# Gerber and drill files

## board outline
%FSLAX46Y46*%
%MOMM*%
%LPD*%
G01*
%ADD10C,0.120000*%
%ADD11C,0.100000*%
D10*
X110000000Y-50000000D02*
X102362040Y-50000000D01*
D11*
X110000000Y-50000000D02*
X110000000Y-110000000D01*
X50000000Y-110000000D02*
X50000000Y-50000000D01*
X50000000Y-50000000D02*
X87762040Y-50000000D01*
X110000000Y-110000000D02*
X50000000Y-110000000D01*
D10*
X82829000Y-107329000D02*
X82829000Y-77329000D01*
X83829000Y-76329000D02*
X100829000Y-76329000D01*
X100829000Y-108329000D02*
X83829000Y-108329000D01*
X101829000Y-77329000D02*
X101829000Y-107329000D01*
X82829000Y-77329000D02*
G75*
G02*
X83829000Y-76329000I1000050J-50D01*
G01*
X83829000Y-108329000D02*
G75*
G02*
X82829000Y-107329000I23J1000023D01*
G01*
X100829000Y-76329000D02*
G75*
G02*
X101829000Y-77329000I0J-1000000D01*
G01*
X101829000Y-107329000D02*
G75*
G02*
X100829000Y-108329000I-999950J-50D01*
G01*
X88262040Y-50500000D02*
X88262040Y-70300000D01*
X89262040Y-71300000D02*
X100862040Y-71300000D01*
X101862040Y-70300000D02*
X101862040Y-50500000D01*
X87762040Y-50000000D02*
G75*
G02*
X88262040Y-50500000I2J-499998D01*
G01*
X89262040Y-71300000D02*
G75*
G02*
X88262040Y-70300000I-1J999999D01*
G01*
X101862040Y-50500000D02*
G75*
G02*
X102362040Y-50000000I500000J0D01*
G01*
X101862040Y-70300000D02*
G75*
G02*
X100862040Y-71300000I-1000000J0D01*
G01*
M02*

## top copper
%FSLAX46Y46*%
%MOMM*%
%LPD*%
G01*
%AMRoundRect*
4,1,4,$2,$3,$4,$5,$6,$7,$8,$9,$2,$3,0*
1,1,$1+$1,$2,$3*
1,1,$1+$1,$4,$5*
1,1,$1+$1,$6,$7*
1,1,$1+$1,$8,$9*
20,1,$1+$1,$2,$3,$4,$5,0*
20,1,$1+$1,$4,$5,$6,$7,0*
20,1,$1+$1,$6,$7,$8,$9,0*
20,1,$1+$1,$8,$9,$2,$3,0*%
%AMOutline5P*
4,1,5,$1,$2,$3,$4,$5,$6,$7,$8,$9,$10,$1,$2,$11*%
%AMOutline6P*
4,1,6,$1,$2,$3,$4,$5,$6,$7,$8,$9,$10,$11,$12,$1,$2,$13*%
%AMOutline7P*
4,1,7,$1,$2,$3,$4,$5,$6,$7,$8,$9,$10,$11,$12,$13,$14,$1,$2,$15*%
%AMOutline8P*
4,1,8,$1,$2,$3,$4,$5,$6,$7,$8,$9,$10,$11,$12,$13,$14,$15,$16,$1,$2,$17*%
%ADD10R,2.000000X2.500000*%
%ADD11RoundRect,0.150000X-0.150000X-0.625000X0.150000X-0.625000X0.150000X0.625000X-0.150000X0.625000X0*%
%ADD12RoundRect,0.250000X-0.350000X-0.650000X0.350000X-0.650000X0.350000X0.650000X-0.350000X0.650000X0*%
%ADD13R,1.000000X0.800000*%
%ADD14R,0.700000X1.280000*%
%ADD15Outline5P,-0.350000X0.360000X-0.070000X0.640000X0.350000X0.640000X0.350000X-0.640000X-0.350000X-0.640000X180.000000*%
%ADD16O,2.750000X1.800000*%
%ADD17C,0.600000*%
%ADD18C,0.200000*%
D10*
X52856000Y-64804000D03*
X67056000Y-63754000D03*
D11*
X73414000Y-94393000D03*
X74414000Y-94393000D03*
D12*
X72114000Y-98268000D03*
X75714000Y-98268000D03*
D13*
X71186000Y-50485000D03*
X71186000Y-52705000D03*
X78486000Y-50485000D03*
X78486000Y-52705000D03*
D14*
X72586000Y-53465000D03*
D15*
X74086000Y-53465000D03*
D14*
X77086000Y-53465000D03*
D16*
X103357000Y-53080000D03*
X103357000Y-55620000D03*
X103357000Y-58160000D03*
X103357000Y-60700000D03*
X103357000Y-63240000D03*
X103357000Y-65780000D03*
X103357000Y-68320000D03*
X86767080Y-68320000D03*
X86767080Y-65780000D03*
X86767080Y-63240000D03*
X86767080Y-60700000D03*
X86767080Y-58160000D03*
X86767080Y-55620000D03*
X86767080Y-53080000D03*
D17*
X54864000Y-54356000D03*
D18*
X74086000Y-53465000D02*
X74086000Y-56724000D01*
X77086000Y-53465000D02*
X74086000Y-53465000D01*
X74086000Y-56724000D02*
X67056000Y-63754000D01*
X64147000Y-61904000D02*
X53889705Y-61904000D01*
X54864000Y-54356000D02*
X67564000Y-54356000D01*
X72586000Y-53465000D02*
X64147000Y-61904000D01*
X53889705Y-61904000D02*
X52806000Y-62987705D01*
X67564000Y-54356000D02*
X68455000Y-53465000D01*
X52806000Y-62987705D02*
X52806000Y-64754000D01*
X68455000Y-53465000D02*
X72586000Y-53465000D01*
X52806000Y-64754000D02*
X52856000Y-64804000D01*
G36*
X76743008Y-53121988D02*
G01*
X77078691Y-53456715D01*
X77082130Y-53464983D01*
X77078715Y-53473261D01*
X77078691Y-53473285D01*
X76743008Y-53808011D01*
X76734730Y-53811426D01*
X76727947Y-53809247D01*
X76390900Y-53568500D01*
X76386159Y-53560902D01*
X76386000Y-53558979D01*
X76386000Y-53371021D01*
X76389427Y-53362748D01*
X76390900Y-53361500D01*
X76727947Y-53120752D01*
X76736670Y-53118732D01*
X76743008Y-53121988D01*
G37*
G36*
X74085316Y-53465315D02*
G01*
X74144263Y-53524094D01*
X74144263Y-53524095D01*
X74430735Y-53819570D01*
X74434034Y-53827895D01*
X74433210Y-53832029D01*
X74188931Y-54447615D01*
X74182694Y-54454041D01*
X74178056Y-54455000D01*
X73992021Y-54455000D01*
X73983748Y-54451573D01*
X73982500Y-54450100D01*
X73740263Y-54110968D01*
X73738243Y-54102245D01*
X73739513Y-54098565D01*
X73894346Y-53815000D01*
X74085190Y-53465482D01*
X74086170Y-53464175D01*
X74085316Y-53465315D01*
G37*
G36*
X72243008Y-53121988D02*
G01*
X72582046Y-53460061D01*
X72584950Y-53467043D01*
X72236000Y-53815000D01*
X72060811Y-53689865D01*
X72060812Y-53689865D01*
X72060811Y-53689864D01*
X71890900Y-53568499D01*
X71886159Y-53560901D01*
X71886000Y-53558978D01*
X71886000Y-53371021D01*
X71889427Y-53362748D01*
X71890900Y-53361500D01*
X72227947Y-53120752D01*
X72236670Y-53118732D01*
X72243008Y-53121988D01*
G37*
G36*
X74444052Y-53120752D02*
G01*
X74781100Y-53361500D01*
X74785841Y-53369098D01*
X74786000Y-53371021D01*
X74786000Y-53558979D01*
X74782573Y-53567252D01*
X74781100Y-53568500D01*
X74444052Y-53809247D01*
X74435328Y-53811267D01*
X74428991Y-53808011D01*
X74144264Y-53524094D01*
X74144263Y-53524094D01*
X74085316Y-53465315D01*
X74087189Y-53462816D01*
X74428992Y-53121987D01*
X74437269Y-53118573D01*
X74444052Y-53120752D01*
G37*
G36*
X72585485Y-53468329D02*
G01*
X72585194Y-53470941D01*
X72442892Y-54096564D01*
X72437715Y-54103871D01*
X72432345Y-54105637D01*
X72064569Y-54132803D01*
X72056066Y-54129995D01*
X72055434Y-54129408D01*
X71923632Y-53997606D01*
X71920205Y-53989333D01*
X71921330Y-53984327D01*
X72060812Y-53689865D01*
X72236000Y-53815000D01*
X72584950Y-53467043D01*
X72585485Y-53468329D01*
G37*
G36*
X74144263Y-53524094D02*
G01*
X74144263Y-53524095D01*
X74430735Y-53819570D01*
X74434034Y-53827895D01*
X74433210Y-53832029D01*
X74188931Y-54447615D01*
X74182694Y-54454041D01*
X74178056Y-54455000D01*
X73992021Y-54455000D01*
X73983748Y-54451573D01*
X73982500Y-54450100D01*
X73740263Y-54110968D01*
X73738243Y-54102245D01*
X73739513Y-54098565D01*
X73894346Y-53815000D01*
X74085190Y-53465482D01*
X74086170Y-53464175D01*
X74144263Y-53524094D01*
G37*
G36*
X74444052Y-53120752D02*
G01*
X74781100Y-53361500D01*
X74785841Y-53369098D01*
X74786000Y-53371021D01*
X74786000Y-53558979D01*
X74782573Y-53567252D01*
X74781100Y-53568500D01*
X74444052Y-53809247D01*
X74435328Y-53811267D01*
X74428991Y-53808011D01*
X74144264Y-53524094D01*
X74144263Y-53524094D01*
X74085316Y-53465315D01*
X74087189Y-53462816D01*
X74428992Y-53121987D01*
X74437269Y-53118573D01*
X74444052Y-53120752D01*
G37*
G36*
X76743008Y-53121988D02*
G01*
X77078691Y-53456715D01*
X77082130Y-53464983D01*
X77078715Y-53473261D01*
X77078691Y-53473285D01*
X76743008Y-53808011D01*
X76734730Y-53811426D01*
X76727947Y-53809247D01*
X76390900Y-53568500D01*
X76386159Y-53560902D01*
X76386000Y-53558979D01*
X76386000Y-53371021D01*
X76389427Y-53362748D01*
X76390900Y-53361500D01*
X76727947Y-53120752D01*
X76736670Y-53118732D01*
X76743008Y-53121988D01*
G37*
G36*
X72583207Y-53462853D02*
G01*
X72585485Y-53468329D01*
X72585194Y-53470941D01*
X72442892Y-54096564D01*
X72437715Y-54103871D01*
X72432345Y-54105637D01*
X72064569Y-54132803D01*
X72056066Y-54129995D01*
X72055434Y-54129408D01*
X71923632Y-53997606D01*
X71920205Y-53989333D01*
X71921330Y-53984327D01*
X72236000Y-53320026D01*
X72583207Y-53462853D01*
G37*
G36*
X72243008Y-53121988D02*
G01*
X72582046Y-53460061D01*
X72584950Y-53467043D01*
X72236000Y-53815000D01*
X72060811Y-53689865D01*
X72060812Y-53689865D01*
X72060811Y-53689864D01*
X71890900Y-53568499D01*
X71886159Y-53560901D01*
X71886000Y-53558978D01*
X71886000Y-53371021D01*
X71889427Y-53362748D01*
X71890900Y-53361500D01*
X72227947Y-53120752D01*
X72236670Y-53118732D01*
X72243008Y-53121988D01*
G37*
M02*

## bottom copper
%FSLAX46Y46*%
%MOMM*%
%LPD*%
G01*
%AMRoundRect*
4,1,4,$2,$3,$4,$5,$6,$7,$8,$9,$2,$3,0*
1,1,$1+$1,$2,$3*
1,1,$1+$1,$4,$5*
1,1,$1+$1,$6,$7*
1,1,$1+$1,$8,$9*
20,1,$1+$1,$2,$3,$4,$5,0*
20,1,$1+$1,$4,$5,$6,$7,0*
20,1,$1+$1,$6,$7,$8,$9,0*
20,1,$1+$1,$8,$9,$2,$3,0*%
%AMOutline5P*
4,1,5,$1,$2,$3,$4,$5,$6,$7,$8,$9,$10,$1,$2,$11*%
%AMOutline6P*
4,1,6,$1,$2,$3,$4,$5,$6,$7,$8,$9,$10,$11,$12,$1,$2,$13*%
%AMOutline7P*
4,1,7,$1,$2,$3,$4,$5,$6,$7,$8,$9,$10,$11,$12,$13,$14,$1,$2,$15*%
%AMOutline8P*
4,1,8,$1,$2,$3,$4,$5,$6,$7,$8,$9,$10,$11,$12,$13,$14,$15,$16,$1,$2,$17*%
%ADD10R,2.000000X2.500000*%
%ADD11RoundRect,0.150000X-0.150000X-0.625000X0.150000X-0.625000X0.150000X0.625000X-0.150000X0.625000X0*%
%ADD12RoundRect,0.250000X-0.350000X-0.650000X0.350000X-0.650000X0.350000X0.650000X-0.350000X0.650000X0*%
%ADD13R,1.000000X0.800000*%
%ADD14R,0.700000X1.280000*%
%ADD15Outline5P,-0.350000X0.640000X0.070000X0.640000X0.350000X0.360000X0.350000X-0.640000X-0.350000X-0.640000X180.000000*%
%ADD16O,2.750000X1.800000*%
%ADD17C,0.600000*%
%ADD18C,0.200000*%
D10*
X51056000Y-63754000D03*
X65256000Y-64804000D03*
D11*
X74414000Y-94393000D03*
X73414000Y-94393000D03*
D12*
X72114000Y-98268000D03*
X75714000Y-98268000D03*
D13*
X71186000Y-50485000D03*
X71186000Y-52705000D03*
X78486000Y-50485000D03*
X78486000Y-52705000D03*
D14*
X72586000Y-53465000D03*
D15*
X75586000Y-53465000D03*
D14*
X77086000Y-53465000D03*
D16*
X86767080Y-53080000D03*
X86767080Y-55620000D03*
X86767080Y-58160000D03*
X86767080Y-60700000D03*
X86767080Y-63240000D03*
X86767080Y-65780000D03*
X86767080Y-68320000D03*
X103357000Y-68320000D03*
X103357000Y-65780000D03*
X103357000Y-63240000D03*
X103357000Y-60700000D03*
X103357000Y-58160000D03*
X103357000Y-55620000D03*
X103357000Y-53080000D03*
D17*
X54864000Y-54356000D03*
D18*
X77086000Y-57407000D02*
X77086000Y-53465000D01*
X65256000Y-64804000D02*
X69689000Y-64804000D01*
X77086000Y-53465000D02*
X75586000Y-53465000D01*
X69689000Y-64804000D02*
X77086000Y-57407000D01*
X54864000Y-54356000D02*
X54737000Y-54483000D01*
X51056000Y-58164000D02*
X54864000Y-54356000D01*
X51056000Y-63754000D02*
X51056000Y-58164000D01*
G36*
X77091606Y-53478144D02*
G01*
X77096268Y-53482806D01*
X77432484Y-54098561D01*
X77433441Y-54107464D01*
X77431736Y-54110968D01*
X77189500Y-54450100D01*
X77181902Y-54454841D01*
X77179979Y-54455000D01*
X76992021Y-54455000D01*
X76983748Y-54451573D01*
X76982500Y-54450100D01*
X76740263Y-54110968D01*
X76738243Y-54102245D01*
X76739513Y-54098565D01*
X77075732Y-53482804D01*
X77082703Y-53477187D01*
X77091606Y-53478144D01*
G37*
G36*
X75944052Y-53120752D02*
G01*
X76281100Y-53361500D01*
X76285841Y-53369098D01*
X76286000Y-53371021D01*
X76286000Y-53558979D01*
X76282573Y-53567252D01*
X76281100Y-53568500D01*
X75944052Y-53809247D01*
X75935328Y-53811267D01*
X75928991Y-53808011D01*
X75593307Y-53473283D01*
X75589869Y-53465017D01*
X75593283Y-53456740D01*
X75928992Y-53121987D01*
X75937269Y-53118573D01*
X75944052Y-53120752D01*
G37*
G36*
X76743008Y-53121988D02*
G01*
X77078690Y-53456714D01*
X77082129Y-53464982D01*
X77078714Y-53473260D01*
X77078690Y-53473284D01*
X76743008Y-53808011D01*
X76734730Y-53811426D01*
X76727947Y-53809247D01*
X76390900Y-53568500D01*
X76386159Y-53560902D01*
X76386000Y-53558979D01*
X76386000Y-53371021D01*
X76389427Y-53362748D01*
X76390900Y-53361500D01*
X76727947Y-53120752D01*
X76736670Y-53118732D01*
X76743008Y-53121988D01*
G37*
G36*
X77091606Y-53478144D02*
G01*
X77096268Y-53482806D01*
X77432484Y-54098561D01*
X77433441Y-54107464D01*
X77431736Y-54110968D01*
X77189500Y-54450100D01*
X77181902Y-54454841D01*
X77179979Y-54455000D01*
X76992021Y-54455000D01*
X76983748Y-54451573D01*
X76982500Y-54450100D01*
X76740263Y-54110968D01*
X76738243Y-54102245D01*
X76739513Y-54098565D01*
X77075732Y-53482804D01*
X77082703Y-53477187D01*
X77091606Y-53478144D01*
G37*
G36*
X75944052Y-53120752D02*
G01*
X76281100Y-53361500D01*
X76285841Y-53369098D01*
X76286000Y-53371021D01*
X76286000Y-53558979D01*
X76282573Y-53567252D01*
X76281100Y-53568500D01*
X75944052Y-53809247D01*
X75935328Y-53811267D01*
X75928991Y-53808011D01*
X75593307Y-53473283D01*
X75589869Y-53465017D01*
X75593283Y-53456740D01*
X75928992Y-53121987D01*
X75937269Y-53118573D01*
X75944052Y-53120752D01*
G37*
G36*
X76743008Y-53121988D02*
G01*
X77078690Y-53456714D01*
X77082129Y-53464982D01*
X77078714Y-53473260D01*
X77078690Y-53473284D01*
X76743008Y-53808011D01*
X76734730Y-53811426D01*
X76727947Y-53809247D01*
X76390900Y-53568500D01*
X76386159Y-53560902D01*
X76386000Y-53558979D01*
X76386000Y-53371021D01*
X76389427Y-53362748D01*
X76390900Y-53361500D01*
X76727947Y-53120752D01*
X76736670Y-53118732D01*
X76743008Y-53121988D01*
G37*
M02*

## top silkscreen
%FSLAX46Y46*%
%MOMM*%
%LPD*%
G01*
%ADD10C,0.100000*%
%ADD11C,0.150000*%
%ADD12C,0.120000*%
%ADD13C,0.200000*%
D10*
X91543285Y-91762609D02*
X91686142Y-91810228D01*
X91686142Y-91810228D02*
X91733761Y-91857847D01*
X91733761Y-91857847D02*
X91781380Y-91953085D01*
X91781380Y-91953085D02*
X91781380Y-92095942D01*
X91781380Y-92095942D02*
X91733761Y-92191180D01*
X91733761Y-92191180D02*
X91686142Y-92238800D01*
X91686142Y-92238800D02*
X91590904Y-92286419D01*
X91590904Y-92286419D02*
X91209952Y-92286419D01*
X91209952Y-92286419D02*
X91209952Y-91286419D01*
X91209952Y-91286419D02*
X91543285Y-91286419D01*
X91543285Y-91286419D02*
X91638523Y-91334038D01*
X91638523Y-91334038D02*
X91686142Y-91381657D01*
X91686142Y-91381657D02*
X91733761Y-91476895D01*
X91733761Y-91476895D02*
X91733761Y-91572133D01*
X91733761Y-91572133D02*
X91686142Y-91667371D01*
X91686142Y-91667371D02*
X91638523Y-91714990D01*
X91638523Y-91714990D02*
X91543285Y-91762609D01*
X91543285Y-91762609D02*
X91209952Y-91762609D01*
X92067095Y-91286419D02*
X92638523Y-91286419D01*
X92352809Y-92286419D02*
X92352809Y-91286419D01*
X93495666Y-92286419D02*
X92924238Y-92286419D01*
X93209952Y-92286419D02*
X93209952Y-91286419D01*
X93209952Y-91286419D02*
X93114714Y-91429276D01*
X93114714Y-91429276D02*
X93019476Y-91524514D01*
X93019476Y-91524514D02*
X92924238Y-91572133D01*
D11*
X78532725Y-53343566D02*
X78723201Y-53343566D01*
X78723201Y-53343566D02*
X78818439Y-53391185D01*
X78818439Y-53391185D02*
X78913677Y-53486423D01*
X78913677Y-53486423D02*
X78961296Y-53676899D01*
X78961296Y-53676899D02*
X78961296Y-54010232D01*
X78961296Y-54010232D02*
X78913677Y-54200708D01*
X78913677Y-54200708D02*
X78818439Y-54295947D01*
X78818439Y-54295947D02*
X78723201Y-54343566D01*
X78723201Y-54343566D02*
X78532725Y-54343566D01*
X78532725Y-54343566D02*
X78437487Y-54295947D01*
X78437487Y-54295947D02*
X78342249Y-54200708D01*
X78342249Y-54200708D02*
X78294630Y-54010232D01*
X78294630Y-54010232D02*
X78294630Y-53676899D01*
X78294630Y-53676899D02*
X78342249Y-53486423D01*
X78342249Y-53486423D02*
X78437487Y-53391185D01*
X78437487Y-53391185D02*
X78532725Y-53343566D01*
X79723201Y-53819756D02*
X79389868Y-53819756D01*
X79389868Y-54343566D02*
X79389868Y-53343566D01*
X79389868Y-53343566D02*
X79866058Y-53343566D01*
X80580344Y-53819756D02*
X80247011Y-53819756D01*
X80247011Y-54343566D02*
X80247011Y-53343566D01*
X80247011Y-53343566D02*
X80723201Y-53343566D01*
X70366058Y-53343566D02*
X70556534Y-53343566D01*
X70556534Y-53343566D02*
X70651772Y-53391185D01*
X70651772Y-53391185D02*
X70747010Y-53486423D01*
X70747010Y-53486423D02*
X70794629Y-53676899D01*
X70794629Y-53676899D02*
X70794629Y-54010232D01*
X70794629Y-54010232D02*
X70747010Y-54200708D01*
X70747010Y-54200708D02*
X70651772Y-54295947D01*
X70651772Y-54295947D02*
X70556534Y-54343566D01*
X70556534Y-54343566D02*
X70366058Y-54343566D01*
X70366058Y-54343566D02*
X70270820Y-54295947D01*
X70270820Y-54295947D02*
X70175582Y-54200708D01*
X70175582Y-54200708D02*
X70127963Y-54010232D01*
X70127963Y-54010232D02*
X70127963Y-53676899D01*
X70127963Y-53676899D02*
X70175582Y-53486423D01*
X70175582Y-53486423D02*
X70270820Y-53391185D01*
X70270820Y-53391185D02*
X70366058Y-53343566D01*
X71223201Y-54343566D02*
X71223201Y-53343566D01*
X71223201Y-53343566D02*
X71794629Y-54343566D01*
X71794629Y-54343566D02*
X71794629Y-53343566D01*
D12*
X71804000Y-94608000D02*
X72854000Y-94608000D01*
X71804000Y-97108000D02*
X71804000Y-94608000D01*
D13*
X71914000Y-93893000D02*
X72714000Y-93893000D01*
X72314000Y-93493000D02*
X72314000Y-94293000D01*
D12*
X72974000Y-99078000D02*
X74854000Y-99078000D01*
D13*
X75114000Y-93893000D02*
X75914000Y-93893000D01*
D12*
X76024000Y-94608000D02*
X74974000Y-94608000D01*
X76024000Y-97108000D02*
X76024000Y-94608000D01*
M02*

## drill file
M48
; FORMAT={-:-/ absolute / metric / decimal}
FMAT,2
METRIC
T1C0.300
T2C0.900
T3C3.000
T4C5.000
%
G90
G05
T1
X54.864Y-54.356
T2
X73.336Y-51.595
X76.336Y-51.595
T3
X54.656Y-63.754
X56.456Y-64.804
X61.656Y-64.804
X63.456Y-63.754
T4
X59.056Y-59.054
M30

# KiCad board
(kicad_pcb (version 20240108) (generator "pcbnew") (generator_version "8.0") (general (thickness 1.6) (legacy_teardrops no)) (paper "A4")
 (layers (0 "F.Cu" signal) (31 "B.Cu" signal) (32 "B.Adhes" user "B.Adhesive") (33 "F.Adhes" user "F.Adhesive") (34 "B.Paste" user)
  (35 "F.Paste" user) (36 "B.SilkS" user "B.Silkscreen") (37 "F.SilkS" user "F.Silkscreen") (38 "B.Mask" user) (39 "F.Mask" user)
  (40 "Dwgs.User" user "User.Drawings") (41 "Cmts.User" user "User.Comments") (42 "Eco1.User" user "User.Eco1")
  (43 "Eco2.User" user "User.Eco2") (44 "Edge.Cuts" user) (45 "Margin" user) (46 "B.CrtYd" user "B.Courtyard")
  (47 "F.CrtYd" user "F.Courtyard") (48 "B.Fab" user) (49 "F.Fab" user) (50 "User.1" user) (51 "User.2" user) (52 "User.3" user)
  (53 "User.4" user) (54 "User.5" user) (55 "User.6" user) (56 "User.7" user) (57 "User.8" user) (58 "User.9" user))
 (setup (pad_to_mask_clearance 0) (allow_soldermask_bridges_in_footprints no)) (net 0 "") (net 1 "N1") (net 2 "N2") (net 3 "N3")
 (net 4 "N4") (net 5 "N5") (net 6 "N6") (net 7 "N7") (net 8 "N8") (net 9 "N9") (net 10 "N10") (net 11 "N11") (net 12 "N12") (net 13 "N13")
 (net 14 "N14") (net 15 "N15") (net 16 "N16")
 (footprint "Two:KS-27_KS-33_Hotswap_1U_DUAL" (layer "F.Cu") (at 59.056 59.054)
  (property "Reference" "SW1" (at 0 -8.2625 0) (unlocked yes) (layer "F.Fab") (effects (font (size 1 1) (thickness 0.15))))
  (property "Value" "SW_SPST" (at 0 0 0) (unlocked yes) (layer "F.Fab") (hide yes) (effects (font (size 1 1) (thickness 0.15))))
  (pad "" np_thru_hole circle (at -4.4 4.7) (size 3 3) (drill 3) (layers "F&B.Cu" "*.Mask"))
  (pad "" np_thru_hole circle (at -2.6 5.75) (size 3 3) (drill 3) (layers "F&B.Cu" "*.Mask"))
  (pad "" np_thru_hole circle (at 0 0) (size 5 5) (drill 5) (layers "F&B.Cu" "*.Mask"))
  (pad "" np_thru_hole circle (at 2.6 5.75) (size 3 3) (drill 3) (layers "F&B.Cu" "*.Mask"))
  (pad "" np_thru_hole circle (at 4.4 4.7) (size 3 3) (drill 3) (layers "F&B.Cu" "*.Mask"))
  (pad "1" smd rect (at -8 4.7) (size 2 2.5) (layers "B.Cu" "B.Paste" "B.Mask") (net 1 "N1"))
  (pad "1" smd rect (at -6.2 5.75) (size 2 2.5) (layers "F.Cu" "F.Paste" "F.Mask") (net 1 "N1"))
  (pad "2" smd rect (at 6.2 5.75) (size 2 2.5) (layers "B.Cu" "B.Paste" "B.Mask") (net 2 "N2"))
  (pad "2" smd rect (at 8 4.7) (size 2 2.5) (layers "F.Cu" "F.Paste" "F.Mask") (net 2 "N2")))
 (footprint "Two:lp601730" (layer "F.Cu") (at 92.329 92.329)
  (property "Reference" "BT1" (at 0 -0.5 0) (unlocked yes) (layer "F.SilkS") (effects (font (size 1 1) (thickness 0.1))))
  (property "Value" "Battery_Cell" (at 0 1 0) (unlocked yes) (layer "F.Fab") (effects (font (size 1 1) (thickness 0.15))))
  (fp_line (start -9.5 15) (end -9.5 -15) (stroke (width 0.12) (type solid)) (layer "Edge.Cuts"))
  (fp_line (start -8.5 -16) (end 8.5 -16) (stroke (width 0.12) (type solid)) (layer "Edge.Cuts"))
  (fp_line (start 8.5 16) (end -8.5 16) (stroke (width 0.12) (type solid)) (layer "Edge.Cuts"))
  (fp_line (start 9.5 -15) (end 9.5 15) (stroke (width 0.12) (type solid)) (layer "Edge.Cuts"))
  (fp_arc (start -9.5 -15) (mid -9.207092 -15.707092) (end -8.5 -16) (stroke (width 0.12) (type default)) (layer "Edge.Cuts"))
  (fp_arc (start -8.5 16) (mid -9.2071 15.7071) (end -9.5 15) (stroke (width 0.12) (type default)) (layer "Edge.Cuts"))
  (fp_arc (start 8.5 -16) (mid 9.207107 -15.707107) (end 9.5 -15) (stroke (width 0.12) (type default)) (layer "Edge.Cuts"))
  (fp_arc (start 9.5 15) (mid 9.207121 15.707121) (end 8.5 16) (stroke (width 0.12) (type default)) (layer "Edge.Cuts")))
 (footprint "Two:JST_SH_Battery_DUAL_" (layer "F.Cu") (at 73.914 96.393)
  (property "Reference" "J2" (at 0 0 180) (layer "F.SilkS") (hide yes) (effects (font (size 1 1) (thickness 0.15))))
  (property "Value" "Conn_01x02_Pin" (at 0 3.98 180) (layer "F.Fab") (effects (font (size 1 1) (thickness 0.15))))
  (fp_line (start -2.11 -1.785) (end -1.06 -1.785) (stroke (width 0.12) (type solid)) (layer "F.SilkS"))
  (fp_line (start -2.11 0.715) (end -2.11 -1.785) (stroke (width 0.12) (type solid)) (layer "F.SilkS"))
  (fp_line (start -2 -2.5) (end -1.2 -2.5) (stroke (width 0.2) (type default)) (layer "F.SilkS"))
  (fp_line (start -1.6 -2.9) (end -1.6 -2.1) (stroke (width 0.2) (type default)) (layer "F.SilkS"))
  (fp_line (start -0.94 2.685) (end 0.94 2.685) (stroke (width 0.12) (type solid)) (layer "F.SilkS"))
  (fp_line (start 1.2 -2.5) (end 2 -2.5) (stroke (width 0.2) (type default)) (layer "F.SilkS"))
  (fp_line (start 2.11 -1.785) (end 1.06 -1.785) (stroke (width 0.12) (type solid)) (layer "F.SilkS"))
  (fp_line (start 2.11 0.715) (end 2.11 -1.785) (stroke (width 0.12) (type solid)) (layer "F.SilkS"))
  (pad "1" smd roundrect (at -0.5 -2) (size 0.6 1.55) (layers "F.Cu" "F.Paste" "F.Mask") (roundrect_rratio 0.25)
   (teardrops (best_length_ratio 0.5) (max_length 1) (best_width_ratio 1) (max_width 2) (curve_points 0) (filter_ratio 0.9) (enabled yes)
    (allow_two_segments yes) (prefer_zone_connections yes)))
  (pad "1" smd roundrect (at 0.5 -2) (size 0.6 1.55) (layers "B.Cu" "B.Paste" "B.Mask") (roundrect_rratio 0.25)
   (teardrops (best_length_ratio 0.5) (max_length 1) (best_width_ratio 1) (max_width 2) (curve_points 0) (filter_ratio 0.9) (enabled yes)
    (allow_two_segments yes) (prefer_zone_connections yes)))
  (pad "2" smd roundrect (at -0.5 -2) (size 0.6 1.55) (layers "B.Cu" "B.Paste" "B.Mask") (roundrect_rratio 0.25)
   (teardrops (best_length_ratio 0.5) (max_length 1) (best_width_ratio 1) (max_width 2) (curve_points 0) (filter_ratio 0.9) (enabled yes)
    (allow_two_segments yes) (prefer_zone_connections yes)))
  (pad "2" smd roundrect (at 0.5 -2) (size 0.6 1.55) (layers "F.Cu" "F.Paste" "F.Mask") (roundrect_rratio 0.25)
   (teardrops (best_length_ratio 0.5) (max_length 1) (best_width_ratio 1) (max_width 2) (curve_points 0) (filter_ratio 0.9) (enabled yes)
    (allow_two_segments yes) (prefer_zone_connections yes)))
  (pad "MP" smd roundrect (at -1.8 1.875) (size 1.2 1.8) (layers "F.Cu" "F.Paste" "F.Mask") (roundrect_rratio 0.208333)
   (teardrops (best_length_ratio 0.5) (max_length 1) (best_width_ratio 1) (max_width 2) (curve_points 0) (filter_ratio 0.9) (enabled yes)
    (allow_two_segments yes) (prefer_zone_connections yes)))
  (pad "MP" smd roundrect (at -1.8 1.875) (size 1.2 1.8) (layers "B.Cu" "B.Paste" "B.Mask") (roundrect_rratio 0.208333)
   (teardrops (best_length_ratio 0.5) (max_length 1) (best_width_ratio 1) (max_width 2) (curve_points 0) (filter_ratio 0.9) (enabled yes)
    (allow_two_segments yes) (prefer_zone_connections yes)))
  (pad "MP" smd roundrect (at 1.8 1.875) (size 1.2 1.8) (layers "F.Cu" "F.Paste" "F.Mask") (roundrect_rratio 0.208333)
   (teardrops (best_length_ratio 0.5) (max_length 1) (best_width_ratio 1) (max_width 2) (curve_points 0) (filter_ratio 0.9) (enabled yes)
    (allow_two_segments yes) (prefer_zone_connections yes)))
  (pad "MP" smd roundrect (at 1.8 1.875) (size 1.2 1.8) (layers "B.Cu" "B.Paste" "B.Mask") (roundrect_rratio 0.208333)
   (teardrops (best_length_ratio 0.5) (max_length 1) (best_width_ratio 1) (max_width 2) (curve_points 0) (filter_ratio 0.9) (enabled yes)
    (allow_two_segments yes) (prefer_zone_connections yes))))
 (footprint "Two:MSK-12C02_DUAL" (layer "F.Cu") (at 74.836 50.325)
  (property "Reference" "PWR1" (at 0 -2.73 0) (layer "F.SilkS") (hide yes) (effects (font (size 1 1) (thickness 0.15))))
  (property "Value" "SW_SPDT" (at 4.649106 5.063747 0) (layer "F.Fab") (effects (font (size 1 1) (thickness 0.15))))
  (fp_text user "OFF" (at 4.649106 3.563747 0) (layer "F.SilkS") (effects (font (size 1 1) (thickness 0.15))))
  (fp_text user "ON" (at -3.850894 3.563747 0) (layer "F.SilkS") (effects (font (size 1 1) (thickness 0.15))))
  (pad "" smd rect (at -3.65 0.16 180) (size 1 0.8) (layers "F.Cu" "F.Paste" "F.Mask")
   (teardrops (best_length_ratio 0.5) (max_length 1) (best_width_ratio 1) (max_width 2) (curve_points 0) (filter_ratio 0.9) (enabled yes)
    (allow_two_segments yes) (prefer_zone_connections yes)))
  (pad "" smd rect (at -3.65 0.16 180) (size 1 0.8) (layers "B.Cu" "B.Paste" "B.Mask")
   (teardrops (best_length_ratio 0.5) (max_length 1) (best_width_ratio 1) (max_width 2) (curve_points 0) (filter_ratio 0.9) (enabled yes)
    (allow_two_segments yes) (prefer_zone_connections yes)))
  (pad "" smd rect (at -3.65 2.38 180) (size 1 0.8) (layers "F.Cu" "F.Paste" "F.Mask")
   (teardrops (best_length_ratio 0.5) (max_length 1) (best_width_ratio 1) (max_width 2) (curve_points 0) (filter_ratio 0.9) (enabled yes)
    (allow_two_segments yes) (prefer_zone_connections yes)))
  (pad "" smd rect (at -3.65 2.38 180) (size 1 0.8) (layers "B.Cu" "B.Paste" "B.Mask")
   (teardrops (best_length_ratio 0.5) (max_length 1) (best_width_ratio 1) (max_width 2) (curve_points 0) (filter_ratio 0.9) (enabled yes)
    (allow_two_segments yes) (prefer_zone_connections yes)))
  (pad "" np_thru_hole circle (at -1.5 1.27 180) (size 0.9 0.9) (drill 0.9) (layers "*.Cu" "*.Mask"))
  (pad "" np_thru_hole circle (at 1.5 1.27 180) (size 0.9 0.9) (drill 0.9) (layers "*.Cu" "*.Mask"))
  (pad "" smd rect (at 3.65 0.16 180) (size 1 0.8) (layers "F.Cu" "F.Paste" "F.Mask")
   (teardrops (best_length_ratio 0.5) (max_length 1) (best_width_ratio 1) (max_width 2) (curve_points 0) (filter_ratio 0.9) (enabled yes)
    (allow_two_segments yes) (prefer_zone_connections yes)))
  (pad "" smd rect (at 3.65 0.16 180) (size 1 0.8) (layers "B.Cu" "B.Paste" "B.Mask")
   (teardrops (best_length_ratio 0.5) (max_length 1) (best_width_ratio 1) (max_width 2) (curve_points 0) (filter_ratio 0.9) (enabled yes)
    (allow_two_segments yes) (prefer_zone_connections yes)))
  (pad "" smd rect (at 3.65 2.38 180) (size 1 0.8) (layers "F.Cu" "F.Paste" "F.Mask")
   (teardrops (best_length_ratio 0.5) (max_length 1) (best_width_ratio 1) (max_width 2) (curve_points 0) (filter_ratio 0.9) (enabled yes)
    (allow_two_segments yes) (prefer_zone_connections yes)))
  (pad "" smd rect (at 3.65 2.38 180) (size 1 0.8) (layers "B.Cu" "B.Paste" "B.Mask")
   (teardrops (best_length_ratio 0.5) (max_length 1) (best_width_ratio 1) (max_width 2) (curve_points 0) (filter_ratio 0.9) (enabled yes)
    (allow_two_segments yes) (prefer_zone_connections yes)))
  (pad "1" smd rect (at -2.25 3.14 180) (size 0.7 1.28) (layers "F.Cu" "F.Paste" "F.Mask") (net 1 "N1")
   (teardrops (best_length_ratio 0.5) (max_length 1) (best_width_ratio 1) (max_width 2) (curve_points 0) (filter_ratio 0.9) (enabled yes)
    (allow_two_segments yes) (prefer_zone_connections yes)))
  (pad "1" smd rect (at -2.25 3.14 180) (size 0.7 1.28) (layers "B.Cu" "B.Paste" "B.Mask") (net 1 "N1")
   (teardrops (best_length_ratio 0.5) (max_length 1) (best_width_ratio 1) (max_width 2) (curve_points 0) (filter_ratio 0.9) (enabled yes)
    (allow_two_segments yes) (prefer_zone_connections yes)))
  (pad "2" smd roundrect (at -0.75 3.14 180) (size 0.7 1.28) (layers "F.Cu" "F.Paste" "F.Mask") (roundrect_rratio 0) (chamfer_ratio 0.4)
   (chamfer top_left) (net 2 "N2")
   (teardrops (best_length_ratio 0.5) (max_length 1) (best_width_ratio 1) (max_width 2) (curve_points 0) (filter_ratio 0.9) (enabled yes)
    (allow_two_segments yes) (prefer_zone_connections yes)))
  (pad "2" smd roundrect (at 0.75 3.14 180) (size 0.7 1.28) (layers "B.Cu" "B.Paste" "B.Mask") (roundrect_rratio 0) (chamfer_ratio 0.4)
   (chamfer top_right) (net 2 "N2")
   (teardrops (best_length_ratio 0.5) (max_length 1) (best_width_ratio 1) (max_width 2) (curve_points 0) (filter_ratio 0.9) (enabled yes)
    (allow_two_segments yes) (prefer_zone_connections yes)))
  (pad "3" smd rect (at 2.25 3.14 180) (size 0.7 1.28) (layers "F.Cu" "F.Paste" "F.Mask") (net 2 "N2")
   (teardrops (best_length_ratio 0.5) (max_length 1) (best_width_ratio 1) (max_width 2) (curve_points 0) (filter_ratio 0.9) (enabled yes)
    (allow_two_segments yes) (prefer_zone_connections yes)))
  (pad "3" smd rect (at 2.25 3.14 180) (size 0.7 1.28) (layers "B.Cu" "B.Paste" "B.Mask") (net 2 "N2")
   (teardrops (best_length_ratio 0.5) (max_length 1) (best_width_ratio 1) (max_width 2) (curve_points 0) (filter_ratio 0.9) (enabled yes)
    (allow_two_segments yes) (prefer_zone_connections yes))))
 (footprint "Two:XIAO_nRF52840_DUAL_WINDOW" (layer "F.Cu") (at 95.06204 50)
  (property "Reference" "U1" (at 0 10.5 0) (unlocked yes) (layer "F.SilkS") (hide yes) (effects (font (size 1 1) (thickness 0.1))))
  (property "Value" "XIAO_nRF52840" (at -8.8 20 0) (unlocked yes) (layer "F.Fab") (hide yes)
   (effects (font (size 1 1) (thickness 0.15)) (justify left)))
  (fp_line (start -6.8 0.5) (end -6.8 20.3) (stroke (width 0.12) (type default)) (layer "Edge.Cuts"))
  (fp_line (start -5.8 21.3) (end 5.8 21.3) (stroke (width 0.12) (type default)) (layer "Edge.Cuts"))
  (fp_line (start 6.8 20.3) (end 6.8 0.5) (stroke (width 0.12) (type default)) (layer "Edge.Cuts"))
  (fp_arc (start -7.3 0) (mid -6.946446 0.146446) (end -6.8 0.5) (stroke (width 0.12) (type default)) (layer "Edge.Cuts"))
  (fp_arc (start -5.8 21.3) (mid -6.507107 21.007107) (end -6.8 20.3) (stroke (width 0.12) (type default)) (layer "Edge.Cuts"))
  (fp_arc (start 6.8 0.5) (mid 6.946447 0.146447) (end 7.3 0) (stroke (width 0.12) (type default)) (layer "Edge.Cuts"))
  (fp_arc (start 6.8 20.3) (mid 6.507107 21.007107) (end 5.8 21.3) (stroke (width 0.12) (type default)) (layer "Edge.Cuts"))
  (pad "1" smd oval (at -8.76996 3.08) (size 2.75 1.8) (drill (offset 0.475 0)) (layers "B.Cu" "B.Paste" "B.Mask") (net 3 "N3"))
  (pad "1" smd oval (at 8.76996 3.08) (size 2.75 1.8) (drill (offset -0.475 0)) (layers "F.Cu" "F.Paste" "F.Mask") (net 3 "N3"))
  (pad "2" smd oval (at -8.76996 5.62) (size 2.75 1.8) (drill (offset 0.475 0)) (layers "B.Cu" "B.Paste" "B.Mask") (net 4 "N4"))
  (pad "2" smd oval (at 8.76996 5.62) (size 2.75 1.8) (drill (offset -0.475 0)) (layers "F.Cu" "F.Paste" "F.Mask") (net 4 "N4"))
  (pad "3" smd oval (at -8.76996 8.16) (size 2.75 1.8) (drill (offset 0.475 0)) (layers "B.Cu" "B.Paste" "B.Mask") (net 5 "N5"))
  (pad "3" smd oval (at 8.76996 8.16) (size 2.75 1.8) (drill (offset -0.475 0)) (layers "F.Cu" "F.Paste" "F.Mask") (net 5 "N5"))
  (pad "4" smd oval (at -8.76996 10.7) (size 2.75 1.8) (drill (offset 0.475 0)) (layers "B.Cu" "B.Paste" "B.Mask") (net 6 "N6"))
  (pad "4" smd oval (at 8.76996 10.7) (size 2.75 1.8) (drill (offset -0.475 0)) (layers "F.Cu" "F.Paste" "F.Mask") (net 6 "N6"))
  (pad "5" smd oval (at -8.76996 13.24) (size 2.75 1.8) (drill (offset 0.475 0)) (layers "B.Cu" "B.Paste" "B.Mask") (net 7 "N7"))
  (pad "5" smd oval (at 8.76996 13.24) (size 2.75 1.8) (drill (offset -0.475 0)) (layers "F.Cu" "F.Paste" "F.Mask") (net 7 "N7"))
  (pad "6" smd oval (at -8.76996 15.78) (size 2.75 1.8) (drill (offset 0.475 0)) (layers "B.Cu" "B.Paste" "B.Mask") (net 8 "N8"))
  (pad "6" smd oval (at 8.76996 15.78) (size 2.75 1.8) (drill (offset -0.475 0)) (layers "F.Cu" "F.Paste" "F.Mask") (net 8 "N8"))
  (pad "7" smd oval (at -8.76996 18.32) (size 2.75 1.8) (drill (offset 0.475 0)) (layers "B.Cu" "B.Paste" "B.Mask") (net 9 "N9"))
  (pad "7" smd oval (at 8.76996 18.32) (size 2.75 1.8) (drill (offset -0.475 0)) (layers "F.Cu" "F.Paste" "F.Mask") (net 9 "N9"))
  (pad "8" smd oval (at -8.76996 18.32 180) (size 2.75 1.8) (drill (offset -0.475 0)) (layers "F.Cu" "F.Paste" "F.Mask") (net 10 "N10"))
  (pad "8" smd oval (at 8.76996 18.32 180) (size 2.75 1.8) (drill (offset 0.475 0)) (layers "B.Cu" "B.Paste" "B.Mask") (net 10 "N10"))
  (pad "9" smd oval (at -8.76996 15.78 180) (size 2.75 1.8) (drill (offset -0.475 0)) (layers "F.Cu" "F.Paste" "F.Mask") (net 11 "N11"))
  (pad "9" smd oval (at 8.76996 15.78 180) (size 2.75 1.8) (drill (offset 0.475 0)) (layers "B.Cu" "B.Paste" "B.Mask") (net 11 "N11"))
  (pad "10" smd oval (at -8.76996 13.24 180) (size 2.75 1.8) (drill (offset -0.475 0)) (layers "F.Cu" "F.Paste" "F.Mask") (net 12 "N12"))
  (pad "10" smd oval (at 8.76996 13.24 180) (size 2.75 1.8) (drill (offset 0.475 0)) (layers "B.Cu" "B.Paste" "B.Mask") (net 12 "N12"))
  (pad "11" smd oval (at -8.76996 10.7 180) (size 2.75 1.8) (drill (offset -0.475 0)) (layers "F.Cu" "F.Paste" "F.Mask") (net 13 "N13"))
  (pad "11" smd oval (at 8.76996 10.7 180) (size 2.75 1.8) (drill (offset 0.475 0)) (layers "B.Cu" "B.Paste" "B.Mask") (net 13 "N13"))
  (pad "12" smd oval (at -8.76996 8.16 180) (size 2.75 1.8) (drill (offset -0.475 0)) (layers "F.Cu" "F.Paste" "F.Mask") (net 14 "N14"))
  (pad "12" smd oval (at 8.76996 8.16 180) (size 2.75 1.8) (drill (offset 0.475 0)) (layers "B.Cu" "B.Paste" "B.Mask") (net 14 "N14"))
  (pad "13" smd oval (at -8.76996 5.62 180) (size 2.75 1.8) (drill (offset -0.475 0)) (layers "F.Cu" "F.Paste" "F.Mask") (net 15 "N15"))
  (pad "13" smd oval (at 8.76996 5.62 180) (size 2.75 1.8) (drill (offset 0.475 0)) (layers "B.Cu" "B.Paste" "B.Mask") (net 15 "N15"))
  (pad "14" smd oval (at -8.76996 3.08 180) (size 2.75 1.8) (drill (offset -0.475 0)) (layers "F.Cu" "F.Paste" "F.Mask") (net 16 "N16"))
  (pad "14" smd oval (at 8.76996 3.08 180) (size 2.75 1.8) (drill (offset 0.475 0)) (layers "B.Cu" "B.Paste" "B.Mask") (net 16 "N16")))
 (gr_line (start 110 50) (end 102.36204 50) (stroke (width 0.12) (type default)) (layer "Edge.Cuts"))
 (gr_line (start 110 50) (end 110 110) (stroke (width 0.1) (type default)) (layer "Edge.Cuts"))
 (gr_line (start 50 110) (end 50 50) (stroke (width 0.1) (type default)) (layer "Edge.Cuts"))
 (gr_line (start 50 50) (end 87.76204 50) (stroke (width 0.1) (type default)) (layer "Edge.Cuts"))
 (gr_line (start 110 110) (end 50 110) (stroke (width 0.1) (type default)) (layer "Edge.Cuts"))
 (segment (start 74.086 53.465) (end 74.086 56.724) (width 0.2) (layer "F.Cu") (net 2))
 (segment (start 77.086 53.465) (end 74.086 53.465) (width 0.2) (layer "F.Cu") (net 2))
 (segment (start 74.086 56.724) (end 67.056 63.754) (width 0.2) (layer "F.Cu") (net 2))
 (segment (start 77.086 57.407) (end 77.086 53.465) (width 0.2) (layer "B.Cu") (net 2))
 (segment (start 65.256 64.804) (end 69.689 64.804) (width 0.2) (layer "B.Cu") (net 2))
 (segment (start 77.086 53.465) (end 75.586 53.465) (width 0.2) (layer "B.Cu") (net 2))
 (segment (start 69.689 64.804) (end 77.086 57.407) (width 0.2) (layer "B.Cu") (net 2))
 (segment (start 64.147 61.904) (end 53.889705 61.904) (width 0.2) (layer "F.Cu") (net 1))
 (segment (start 54.864 54.356) (end 67.564 54.356) (width 0.2) (layer "F.Cu") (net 1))
 (segment (start 72.586 53.465) (end 64.147 61.904) (width 0.2) (layer "F.Cu") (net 1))
 (segment (start 53.889705 61.904) (end 52.806 62.987705) (width 0.2) (layer "F.Cu") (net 1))
 (segment (start 67.564 54.356) (end 68.455 53.465) (width 0.2) (layer "F.Cu") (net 1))
 (segment (start 52.806 62.987705) (end 52.806 64.754) (width 0.2) (layer "F.Cu") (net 1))
 (segment (start 68.455 53.465) (end 72.586 53.465) (width 0.2) (layer "F.Cu") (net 1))
 (segment (start 52.806 64.754) (end 52.856 64.804) (width 0.2) (layer "F.Cu") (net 1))
 (via (at 54.864 54.356) (size 0.6) (drill 0.3) (layers "F.Cu" "B.Cu") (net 1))
 (segment (start 54.864 54.356) (end 54.737 54.483) (width 0.2) (layer "B.Cu") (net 1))
 (segment (start 51.056 58.164) (end 54.864 54.356) (width 0.2) (layer "B.Cu") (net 1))
 (segment (start 51.056 63.754) (end 51.056 58.164) (width 0.2) (layer "B.Cu") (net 1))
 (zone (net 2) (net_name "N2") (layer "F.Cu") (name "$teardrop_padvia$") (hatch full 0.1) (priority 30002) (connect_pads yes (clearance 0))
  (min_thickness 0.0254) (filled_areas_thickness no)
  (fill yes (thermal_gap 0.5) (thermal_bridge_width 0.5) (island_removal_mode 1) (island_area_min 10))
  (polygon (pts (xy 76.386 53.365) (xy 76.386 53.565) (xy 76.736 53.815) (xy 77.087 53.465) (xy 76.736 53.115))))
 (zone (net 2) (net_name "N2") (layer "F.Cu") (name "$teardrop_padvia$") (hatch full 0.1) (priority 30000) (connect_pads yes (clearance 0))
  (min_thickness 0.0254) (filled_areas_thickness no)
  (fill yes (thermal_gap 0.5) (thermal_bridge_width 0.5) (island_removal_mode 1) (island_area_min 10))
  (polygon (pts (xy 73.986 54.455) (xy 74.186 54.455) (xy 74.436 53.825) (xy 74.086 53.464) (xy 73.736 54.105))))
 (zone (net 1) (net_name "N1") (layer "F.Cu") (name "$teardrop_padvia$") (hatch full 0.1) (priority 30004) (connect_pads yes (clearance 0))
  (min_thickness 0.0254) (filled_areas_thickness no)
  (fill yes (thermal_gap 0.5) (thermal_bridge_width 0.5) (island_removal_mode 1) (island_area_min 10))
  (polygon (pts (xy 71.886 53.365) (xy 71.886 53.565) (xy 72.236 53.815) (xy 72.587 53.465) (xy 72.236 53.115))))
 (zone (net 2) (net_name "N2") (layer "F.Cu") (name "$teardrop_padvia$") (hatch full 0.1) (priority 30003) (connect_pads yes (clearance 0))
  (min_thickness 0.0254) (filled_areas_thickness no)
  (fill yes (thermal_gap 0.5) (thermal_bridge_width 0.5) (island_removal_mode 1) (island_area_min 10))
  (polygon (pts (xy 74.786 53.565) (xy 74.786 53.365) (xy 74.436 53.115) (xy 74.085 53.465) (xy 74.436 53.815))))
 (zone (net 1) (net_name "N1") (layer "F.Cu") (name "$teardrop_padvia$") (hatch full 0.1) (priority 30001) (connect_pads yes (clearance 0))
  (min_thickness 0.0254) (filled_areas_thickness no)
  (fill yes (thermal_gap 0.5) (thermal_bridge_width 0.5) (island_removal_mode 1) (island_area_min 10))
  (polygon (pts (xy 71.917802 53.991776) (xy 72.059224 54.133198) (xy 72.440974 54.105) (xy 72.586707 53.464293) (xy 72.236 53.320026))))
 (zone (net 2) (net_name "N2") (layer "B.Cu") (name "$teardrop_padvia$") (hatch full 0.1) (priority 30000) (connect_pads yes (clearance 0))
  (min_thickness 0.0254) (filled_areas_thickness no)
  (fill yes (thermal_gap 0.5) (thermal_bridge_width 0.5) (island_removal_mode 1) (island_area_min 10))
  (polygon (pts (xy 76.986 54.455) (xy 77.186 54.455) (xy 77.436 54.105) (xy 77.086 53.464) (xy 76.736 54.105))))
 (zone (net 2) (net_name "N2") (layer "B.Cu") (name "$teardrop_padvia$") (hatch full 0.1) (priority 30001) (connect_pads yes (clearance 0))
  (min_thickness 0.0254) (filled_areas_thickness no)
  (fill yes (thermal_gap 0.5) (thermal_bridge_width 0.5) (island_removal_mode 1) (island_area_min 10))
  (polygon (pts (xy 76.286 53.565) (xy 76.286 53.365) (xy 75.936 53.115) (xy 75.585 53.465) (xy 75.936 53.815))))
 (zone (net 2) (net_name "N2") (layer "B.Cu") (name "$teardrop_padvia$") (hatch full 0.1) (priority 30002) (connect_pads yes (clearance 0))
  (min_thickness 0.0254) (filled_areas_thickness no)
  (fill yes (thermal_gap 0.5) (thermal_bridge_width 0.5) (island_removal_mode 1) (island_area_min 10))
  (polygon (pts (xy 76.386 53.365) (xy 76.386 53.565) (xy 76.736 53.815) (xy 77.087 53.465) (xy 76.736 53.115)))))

